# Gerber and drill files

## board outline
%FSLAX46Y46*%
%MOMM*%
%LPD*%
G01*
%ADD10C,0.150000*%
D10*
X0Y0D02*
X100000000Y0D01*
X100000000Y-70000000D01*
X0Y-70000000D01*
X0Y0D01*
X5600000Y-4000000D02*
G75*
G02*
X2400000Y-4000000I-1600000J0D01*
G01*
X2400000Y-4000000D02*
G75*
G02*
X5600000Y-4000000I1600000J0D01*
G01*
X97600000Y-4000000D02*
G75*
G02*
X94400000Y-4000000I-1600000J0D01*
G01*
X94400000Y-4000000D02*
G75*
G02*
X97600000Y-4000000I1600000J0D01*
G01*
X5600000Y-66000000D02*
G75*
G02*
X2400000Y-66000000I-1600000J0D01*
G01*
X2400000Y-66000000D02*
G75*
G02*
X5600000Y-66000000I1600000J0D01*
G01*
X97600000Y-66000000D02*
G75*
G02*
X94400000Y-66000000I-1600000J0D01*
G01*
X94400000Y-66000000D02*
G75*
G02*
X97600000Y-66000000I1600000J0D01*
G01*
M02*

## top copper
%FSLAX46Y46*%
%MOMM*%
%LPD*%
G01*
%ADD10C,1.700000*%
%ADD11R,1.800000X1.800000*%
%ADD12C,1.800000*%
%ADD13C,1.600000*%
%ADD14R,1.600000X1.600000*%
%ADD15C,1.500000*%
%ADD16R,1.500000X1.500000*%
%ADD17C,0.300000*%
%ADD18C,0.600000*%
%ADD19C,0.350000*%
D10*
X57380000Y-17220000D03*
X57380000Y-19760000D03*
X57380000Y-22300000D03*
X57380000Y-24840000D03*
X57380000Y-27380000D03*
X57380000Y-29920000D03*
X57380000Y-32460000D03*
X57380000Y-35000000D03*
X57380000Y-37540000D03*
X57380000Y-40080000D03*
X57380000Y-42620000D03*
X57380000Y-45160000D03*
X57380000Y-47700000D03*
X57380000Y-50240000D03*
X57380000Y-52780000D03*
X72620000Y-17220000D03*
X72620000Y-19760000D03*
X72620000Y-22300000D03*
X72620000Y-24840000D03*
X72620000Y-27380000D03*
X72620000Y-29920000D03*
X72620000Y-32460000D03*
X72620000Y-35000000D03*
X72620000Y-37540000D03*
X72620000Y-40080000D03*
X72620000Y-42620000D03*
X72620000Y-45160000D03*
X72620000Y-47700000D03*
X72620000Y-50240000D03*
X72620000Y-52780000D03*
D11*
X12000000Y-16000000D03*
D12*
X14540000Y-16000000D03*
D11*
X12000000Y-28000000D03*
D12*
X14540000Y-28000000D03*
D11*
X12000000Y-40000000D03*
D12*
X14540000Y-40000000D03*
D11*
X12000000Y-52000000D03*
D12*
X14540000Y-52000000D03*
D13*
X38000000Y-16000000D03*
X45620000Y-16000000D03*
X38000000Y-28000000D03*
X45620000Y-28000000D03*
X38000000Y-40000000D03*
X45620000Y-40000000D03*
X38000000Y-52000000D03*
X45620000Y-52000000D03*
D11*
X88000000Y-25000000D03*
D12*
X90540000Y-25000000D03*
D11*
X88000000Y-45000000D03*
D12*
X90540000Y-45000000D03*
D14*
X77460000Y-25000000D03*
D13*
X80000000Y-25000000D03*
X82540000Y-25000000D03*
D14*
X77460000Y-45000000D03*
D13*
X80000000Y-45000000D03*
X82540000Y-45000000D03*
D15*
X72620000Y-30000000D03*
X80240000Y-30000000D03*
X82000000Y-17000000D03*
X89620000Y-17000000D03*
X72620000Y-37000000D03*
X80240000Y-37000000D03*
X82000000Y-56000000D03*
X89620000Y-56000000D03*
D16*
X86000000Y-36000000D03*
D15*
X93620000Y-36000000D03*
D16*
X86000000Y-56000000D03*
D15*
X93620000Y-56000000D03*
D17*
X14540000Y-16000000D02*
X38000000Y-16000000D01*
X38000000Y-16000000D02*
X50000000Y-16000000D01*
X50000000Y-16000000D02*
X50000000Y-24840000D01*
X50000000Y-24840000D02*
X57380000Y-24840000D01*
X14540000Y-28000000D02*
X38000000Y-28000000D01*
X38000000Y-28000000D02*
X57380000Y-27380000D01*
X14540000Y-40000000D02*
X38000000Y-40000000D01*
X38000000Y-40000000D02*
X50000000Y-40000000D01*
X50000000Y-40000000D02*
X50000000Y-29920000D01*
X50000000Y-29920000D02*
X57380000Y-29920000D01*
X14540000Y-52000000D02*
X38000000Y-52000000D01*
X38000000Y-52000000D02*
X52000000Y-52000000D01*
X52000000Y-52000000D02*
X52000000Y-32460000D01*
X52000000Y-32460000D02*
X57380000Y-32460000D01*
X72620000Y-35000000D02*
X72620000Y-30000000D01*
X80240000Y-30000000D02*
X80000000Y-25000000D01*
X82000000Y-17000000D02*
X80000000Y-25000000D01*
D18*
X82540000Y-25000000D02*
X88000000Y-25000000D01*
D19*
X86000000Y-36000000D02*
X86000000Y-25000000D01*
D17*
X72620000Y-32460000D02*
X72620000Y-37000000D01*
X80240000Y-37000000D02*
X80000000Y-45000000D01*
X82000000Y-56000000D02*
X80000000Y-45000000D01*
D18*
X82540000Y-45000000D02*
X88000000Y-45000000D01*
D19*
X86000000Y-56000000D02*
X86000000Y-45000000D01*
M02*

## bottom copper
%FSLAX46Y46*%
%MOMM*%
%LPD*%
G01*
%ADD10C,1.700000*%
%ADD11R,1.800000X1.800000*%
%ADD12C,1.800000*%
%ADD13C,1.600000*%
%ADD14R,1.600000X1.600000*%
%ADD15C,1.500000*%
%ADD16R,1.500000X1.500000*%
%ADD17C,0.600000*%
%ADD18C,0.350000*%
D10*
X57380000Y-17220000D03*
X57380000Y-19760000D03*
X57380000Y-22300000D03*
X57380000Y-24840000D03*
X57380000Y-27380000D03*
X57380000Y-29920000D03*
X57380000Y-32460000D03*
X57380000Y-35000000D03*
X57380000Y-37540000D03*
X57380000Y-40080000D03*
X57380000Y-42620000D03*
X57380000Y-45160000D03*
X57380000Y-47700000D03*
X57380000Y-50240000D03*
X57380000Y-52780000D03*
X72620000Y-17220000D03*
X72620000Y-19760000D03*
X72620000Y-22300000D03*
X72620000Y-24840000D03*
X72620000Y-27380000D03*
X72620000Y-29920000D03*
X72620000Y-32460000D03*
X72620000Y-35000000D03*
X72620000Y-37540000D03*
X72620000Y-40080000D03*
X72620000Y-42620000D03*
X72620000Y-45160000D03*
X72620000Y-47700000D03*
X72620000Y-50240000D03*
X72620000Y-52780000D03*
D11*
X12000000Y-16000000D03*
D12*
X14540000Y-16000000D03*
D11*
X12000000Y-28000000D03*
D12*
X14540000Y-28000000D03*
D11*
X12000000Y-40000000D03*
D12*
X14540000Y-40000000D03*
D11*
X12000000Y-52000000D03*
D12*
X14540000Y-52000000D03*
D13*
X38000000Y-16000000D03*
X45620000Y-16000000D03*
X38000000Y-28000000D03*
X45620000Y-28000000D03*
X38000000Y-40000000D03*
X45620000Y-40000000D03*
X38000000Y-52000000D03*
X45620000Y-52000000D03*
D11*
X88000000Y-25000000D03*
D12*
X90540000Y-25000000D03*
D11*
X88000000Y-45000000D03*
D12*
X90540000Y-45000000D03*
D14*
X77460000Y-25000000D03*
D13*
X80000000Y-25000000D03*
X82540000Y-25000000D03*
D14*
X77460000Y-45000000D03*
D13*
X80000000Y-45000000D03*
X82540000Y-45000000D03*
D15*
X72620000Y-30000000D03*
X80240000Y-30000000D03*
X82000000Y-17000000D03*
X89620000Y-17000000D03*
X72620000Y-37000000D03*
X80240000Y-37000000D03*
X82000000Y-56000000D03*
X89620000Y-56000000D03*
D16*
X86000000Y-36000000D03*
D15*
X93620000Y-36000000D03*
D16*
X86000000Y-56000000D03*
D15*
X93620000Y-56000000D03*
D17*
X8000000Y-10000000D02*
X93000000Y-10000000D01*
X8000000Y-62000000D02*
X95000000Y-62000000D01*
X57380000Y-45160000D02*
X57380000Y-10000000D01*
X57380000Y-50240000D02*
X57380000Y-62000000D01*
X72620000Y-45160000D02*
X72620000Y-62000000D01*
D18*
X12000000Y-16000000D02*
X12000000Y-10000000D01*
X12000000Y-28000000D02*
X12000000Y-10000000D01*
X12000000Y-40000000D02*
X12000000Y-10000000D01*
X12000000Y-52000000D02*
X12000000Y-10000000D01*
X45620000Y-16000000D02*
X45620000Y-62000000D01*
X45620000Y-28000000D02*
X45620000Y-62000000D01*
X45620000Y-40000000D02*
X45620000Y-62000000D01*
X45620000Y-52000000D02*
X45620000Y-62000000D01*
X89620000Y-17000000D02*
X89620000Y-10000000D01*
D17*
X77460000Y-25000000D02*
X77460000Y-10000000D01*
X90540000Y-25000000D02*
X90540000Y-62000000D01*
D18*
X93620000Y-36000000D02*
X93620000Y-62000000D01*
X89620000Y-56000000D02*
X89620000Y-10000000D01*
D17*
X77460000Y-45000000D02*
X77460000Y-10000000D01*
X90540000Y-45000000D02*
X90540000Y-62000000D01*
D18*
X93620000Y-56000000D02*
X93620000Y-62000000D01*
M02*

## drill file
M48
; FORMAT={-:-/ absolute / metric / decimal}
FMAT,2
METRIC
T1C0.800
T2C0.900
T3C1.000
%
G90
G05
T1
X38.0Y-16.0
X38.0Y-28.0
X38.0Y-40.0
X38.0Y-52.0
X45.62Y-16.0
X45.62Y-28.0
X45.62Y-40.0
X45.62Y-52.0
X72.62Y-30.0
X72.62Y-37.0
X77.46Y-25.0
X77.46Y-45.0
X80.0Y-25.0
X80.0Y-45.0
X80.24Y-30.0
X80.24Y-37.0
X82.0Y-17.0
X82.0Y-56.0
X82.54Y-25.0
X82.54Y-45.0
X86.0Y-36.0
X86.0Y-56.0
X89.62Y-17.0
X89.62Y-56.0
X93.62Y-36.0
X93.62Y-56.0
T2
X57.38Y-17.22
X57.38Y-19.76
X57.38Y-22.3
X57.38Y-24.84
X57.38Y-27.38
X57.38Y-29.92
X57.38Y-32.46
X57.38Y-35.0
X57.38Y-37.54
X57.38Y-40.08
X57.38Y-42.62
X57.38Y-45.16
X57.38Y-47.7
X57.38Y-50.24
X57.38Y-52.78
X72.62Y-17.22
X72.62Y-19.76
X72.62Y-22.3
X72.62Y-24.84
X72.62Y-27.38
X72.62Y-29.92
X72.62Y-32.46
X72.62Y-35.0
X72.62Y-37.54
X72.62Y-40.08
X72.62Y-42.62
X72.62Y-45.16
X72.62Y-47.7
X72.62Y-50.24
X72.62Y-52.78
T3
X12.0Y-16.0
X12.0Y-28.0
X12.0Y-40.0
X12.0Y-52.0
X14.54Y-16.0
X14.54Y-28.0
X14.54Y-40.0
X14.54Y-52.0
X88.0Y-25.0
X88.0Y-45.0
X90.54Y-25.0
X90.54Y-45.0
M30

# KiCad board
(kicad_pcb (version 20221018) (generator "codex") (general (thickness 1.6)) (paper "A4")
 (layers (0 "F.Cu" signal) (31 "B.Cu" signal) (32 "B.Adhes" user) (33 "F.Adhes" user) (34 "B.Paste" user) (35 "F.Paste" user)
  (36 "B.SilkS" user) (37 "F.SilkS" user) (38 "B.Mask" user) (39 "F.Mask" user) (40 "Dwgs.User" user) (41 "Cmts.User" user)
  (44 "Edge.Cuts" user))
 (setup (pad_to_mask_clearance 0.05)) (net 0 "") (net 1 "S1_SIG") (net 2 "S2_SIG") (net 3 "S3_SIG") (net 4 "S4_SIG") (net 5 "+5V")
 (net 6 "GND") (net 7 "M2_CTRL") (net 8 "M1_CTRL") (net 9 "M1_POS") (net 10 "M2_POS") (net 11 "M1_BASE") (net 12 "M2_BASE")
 (gr_rect (start 0 0) (end 100 70) (stroke (width 0.15) (type default)) (fill none) (layer "Edge.Cuts"))
 (gr_circle (center 4 4) (end 5.6 4) (stroke (width 0.15) (type default)) (fill none) (layer "Edge.Cuts"))
 (gr_circle (center 96 4) (end 97.6 4) (stroke (width 0.15) (type default)) (fill none) (layer "Edge.Cuts"))
 (gr_circle (center 4 66) (end 5.6 66) (stroke (width 0.15) (type default)) (fill none) (layer "Edge.Cuts"))
 (gr_circle (center 96 66) (end 97.6 66) (stroke (width 0.15) (type default)) (fill none) (layer "Edge.Cuts"))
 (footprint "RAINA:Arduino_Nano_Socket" (layer "F.Cu") (at 0 0)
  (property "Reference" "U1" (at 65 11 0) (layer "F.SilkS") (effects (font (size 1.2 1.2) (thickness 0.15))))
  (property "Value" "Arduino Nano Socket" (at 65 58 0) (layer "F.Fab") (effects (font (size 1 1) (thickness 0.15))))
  (pad "L1" thru_hole circle (at 57.38 17.22) (size 1.7 1.7) (drill 0.9) (layers "*.Cu" "*.Mask") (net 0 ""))
  (pad "L2" thru_hole circle (at 57.38 19.76) (size 1.7 1.7) (drill 0.9) (layers "*.Cu" "*.Mask") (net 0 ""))
  (pad "L3" thru_hole circle (at 57.38 22.30) (size 1.7 1.7) (drill 0.9) (layers "*.Cu" "*.Mask") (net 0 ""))
  (pad "L4" thru_hole circle (at 57.38 24.84) (size 1.7 1.7) (drill 0.9) (layers "*.Cu" "*.Mask") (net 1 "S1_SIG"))
  (pad "L5" thru_hole circle (at 57.38 27.38) (size 1.7 1.7) (drill 0.9) (layers "*.Cu" "*.Mask") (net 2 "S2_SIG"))
  (pad "L6" thru_hole circle (at 57.38 29.92) (size 1.7 1.7) (drill 0.9) (layers "*.Cu" "*.Mask") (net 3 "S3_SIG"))
  (pad "L7" thru_hole circle (at 57.38 32.46) (size 1.7 1.7) (drill 0.9) (layers "*.Cu" "*.Mask") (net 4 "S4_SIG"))
  (pad "L8" thru_hole circle (at 57.38 35.00) (size 1.7 1.7) (drill 0.9) (layers "*.Cu" "*.Mask") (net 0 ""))
  (pad "L9" thru_hole circle (at 57.38 37.54) (size 1.7 1.7) (drill 0.9) (layers "*.Cu" "*.Mask") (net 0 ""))
  (pad "L10" thru_hole circle (at 57.38 40.08) (size 1.7 1.7) (drill 0.9) (layers "*.Cu" "*.Mask") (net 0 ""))
  (pad "L11" thru_hole circle (at 57.38 42.62) (size 1.7 1.7) (drill 0.9) (layers "*.Cu" "*.Mask") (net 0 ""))
  (pad "L12" thru_hole circle (at 57.38 45.16) (size 1.7 1.7) (drill 0.9) (layers "*.Cu" "*.Mask") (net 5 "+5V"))
  (pad "L13" thru_hole circle (at 57.38 47.70) (size 1.7 1.7) (drill 0.9) (layers "*.Cu" "*.Mask") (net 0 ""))
  (pad "L14" thru_hole circle (at 57.38 50.24) (size 1.7 1.7) (drill 0.9) (layers "*.Cu" "*.Mask") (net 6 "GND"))
  (pad "L15" thru_hole circle (at 57.38 52.78) (size 1.7 1.7) (drill 0.9) (layers "*.Cu" "*.Mask") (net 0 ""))
  (pad "R1" thru_hole circle (at 72.62 17.22) (size 1.7 1.7) (drill 0.9) (layers "*.Cu" "*.Mask") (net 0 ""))
  (pad "R2" thru_hole circle (at 72.62 19.76) (size 1.7 1.7) (drill 0.9) (layers "*.Cu" "*.Mask") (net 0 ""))
  (pad "R3" thru_hole circle (at 72.62 22.30) (size 1.7 1.7) (drill 0.9) (layers "*.Cu" "*.Mask") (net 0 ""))
  (pad "R4" thru_hole circle (at 72.62 24.84) (size 1.7 1.7) (drill 0.9) (layers "*.Cu" "*.Mask") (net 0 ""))
  (pad "R5" thru_hole circle (at 72.62 27.38) (size 1.7 1.7) (drill 0.9) (layers "*.Cu" "*.Mask") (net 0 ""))
  (pad "R6" thru_hole circle (at 72.62 29.92) (size 1.7 1.7) (drill 0.9) (layers "*.Cu" "*.Mask") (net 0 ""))
  (pad "R7" thru_hole circle (at 72.62 32.46) (size 1.7 1.7) (drill 0.9) (layers "*.Cu" "*.Mask") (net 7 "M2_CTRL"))
  (pad "R8" thru_hole circle (at 72.62 35.00) (size 1.7 1.7) (drill 0.9) (layers "*.Cu" "*.Mask") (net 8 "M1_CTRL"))
  (pad "R9" thru_hole circle (at 72.62 37.54) (size 1.7 1.7) (drill 0.9) (layers "*.Cu" "*.Mask") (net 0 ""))
  (pad "R10" thru_hole circle (at 72.62 40.08) (size 1.7 1.7) (drill 0.9) (layers "*.Cu" "*.Mask") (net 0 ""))
  (pad "R11" thru_hole circle (at 72.62 42.62) (size 1.7 1.7) (drill 0.9) (layers "*.Cu" "*.Mask") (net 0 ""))
  (pad "R12" thru_hole circle (at 72.62 45.16) (size 1.7 1.7) (drill 0.9) (layers "*.Cu" "*.Mask") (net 6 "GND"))
  (pad "R13" thru_hole circle (at 72.62 47.70) (size 1.7 1.7) (drill 0.9) (layers "*.Cu" "*.Mask") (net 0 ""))
  (pad "R14" thru_hole circle (at 72.62 50.24) (size 1.7 1.7) (drill 0.9) (layers "*.Cu" "*.Mask") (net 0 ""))
  (pad "R15" thru_hole circle (at 72.62 52.78) (size 1.7 1.7) (drill 0.9) (layers "*.Cu" "*.Mask") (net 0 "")))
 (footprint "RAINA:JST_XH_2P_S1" (layer "F.Cu") (at 0 0)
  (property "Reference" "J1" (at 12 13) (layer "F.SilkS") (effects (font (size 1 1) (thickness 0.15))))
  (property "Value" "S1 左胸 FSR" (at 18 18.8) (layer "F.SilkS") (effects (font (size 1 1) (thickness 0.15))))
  (pad "1" thru_hole rect (at 12 16) (size 1.8 1.8) (drill 1.0) (layers "*.Cu" "*.Mask") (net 5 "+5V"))
  (pad "2" thru_hole circle (at 14.54 16) (size 1.8 1.8) (drill 1.0) (layers "*.Cu" "*.Mask") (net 1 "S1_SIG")))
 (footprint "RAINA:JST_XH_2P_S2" (layer "F.Cu") (at 0 0)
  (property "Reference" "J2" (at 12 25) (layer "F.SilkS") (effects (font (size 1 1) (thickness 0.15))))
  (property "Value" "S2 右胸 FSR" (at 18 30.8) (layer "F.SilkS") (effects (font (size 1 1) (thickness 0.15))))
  (pad "1" thru_hole rect (at 12 28) (size 1.8 1.8) (drill 1.0) (layers "*.Cu" "*.Mask") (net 5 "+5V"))
  (pad "2" thru_hole circle (at 14.54 28) (size 1.8 1.8) (drill 1.0) (layers "*.Cu" "*.Mask") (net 2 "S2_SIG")))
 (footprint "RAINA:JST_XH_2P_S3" (layer "F.Cu") (at 0 0)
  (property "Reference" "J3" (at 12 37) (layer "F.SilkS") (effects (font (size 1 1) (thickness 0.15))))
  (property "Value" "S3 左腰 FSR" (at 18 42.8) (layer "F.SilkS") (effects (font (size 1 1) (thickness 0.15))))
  (pad "1" thru_hole rect (at 12 40) (size 1.8 1.8) (drill 1.0) (layers "*.Cu" "*.Mask") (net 5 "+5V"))
  (pad "2" thru_hole circle (at 14.54 40) (size 1.8 1.8) (drill 1.0) (layers "*.Cu" "*.Mask") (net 3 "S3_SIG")))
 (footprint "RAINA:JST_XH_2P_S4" (layer "F.Cu") (at 0 0)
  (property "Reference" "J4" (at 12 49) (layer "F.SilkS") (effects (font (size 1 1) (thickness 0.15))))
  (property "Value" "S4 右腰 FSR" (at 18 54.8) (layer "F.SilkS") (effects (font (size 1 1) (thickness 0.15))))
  (pad "1" thru_hole rect (at 12 52) (size 1.8 1.8) (drill 1.0) (layers "*.Cu" "*.Mask") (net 5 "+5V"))
  (pad "2" thru_hole circle (at 14.54 52) (size 1.8 1.8) (drill 1.0) (layers "*.Cu" "*.Mask") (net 4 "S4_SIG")))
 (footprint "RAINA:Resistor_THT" (layer "F.Cu") (at 0 0)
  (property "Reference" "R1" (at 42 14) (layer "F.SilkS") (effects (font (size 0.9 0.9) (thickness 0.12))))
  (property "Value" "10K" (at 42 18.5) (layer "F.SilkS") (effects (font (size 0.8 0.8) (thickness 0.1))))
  (pad "1" thru_hole circle (at 38 16) (size 1.6 1.6) (drill 0.8) (layers "*.Cu" "*.Mask") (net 1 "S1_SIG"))
  (pad "2" thru_hole circle (at 45.62 16) (size 1.6 1.6) (drill 0.8) (layers "*.Cu" "*.Mask") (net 6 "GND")))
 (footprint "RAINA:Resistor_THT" (layer "F.Cu") (at 0 0)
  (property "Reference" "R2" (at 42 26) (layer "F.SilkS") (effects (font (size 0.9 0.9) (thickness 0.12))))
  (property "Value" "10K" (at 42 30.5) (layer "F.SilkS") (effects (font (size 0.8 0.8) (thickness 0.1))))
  (pad "1" thru_hole circle (at 38 28) (size 1.6 1.6) (drill 0.8) (layers "*.Cu" "*.Mask") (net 2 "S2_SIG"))
  (pad "2" thru_hole circle (at 45.62 28) (size 1.6 1.6) (drill 0.8) (layers "*.Cu" "*.Mask") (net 6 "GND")))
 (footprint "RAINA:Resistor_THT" (layer "F.Cu") (at 0 0)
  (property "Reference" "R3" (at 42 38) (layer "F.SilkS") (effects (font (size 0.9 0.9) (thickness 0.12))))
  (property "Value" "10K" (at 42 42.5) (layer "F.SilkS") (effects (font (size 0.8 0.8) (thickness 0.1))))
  (pad "1" thru_hole circle (at 38 40) (size 1.6 1.6) (drill 0.8) (layers "*.Cu" "*.Mask") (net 3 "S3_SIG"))
  (pad "2" thru_hole circle (at 45.62 40) (size 1.6 1.6) (drill 0.8) (layers "*.Cu" "*.Mask") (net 6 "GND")))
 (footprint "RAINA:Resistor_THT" (layer "F.Cu") (at 0 0)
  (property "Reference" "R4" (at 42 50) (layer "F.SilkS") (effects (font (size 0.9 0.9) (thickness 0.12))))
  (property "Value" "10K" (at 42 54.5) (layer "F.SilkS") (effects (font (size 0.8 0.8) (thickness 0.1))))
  (pad "1" thru_hole circle (at 38 52) (size 1.6 1.6) (drill 0.8) (layers "*.Cu" "*.Mask") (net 4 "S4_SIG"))
  (pad "2" thru_hole circle (at 45.62 52) (size 1.6 1.6) (drill 0.8) (layers "*.Cu" "*.Mask") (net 6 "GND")))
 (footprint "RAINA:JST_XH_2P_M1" (layer "F.Cu") (at 0 0)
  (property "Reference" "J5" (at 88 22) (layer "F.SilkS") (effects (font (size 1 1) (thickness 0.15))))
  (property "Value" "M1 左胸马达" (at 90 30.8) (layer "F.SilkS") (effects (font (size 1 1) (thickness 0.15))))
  (pad "1" thru_hole rect (at 88 25) (size 1.8 1.8) (drill 1.0) (layers "*.Cu" "*.Mask") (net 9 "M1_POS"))
  (pad "2" thru_hole circle (at 90.54 25) (size 1.8 1.8) (drill 1.0) (layers "*.Cu" "*.Mask") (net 6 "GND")))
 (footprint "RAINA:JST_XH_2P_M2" (layer "F.Cu") (at 0 0)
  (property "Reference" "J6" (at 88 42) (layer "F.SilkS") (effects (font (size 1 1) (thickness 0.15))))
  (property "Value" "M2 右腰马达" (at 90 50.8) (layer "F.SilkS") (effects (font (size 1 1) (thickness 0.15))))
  (pad "1" thru_hole rect (at 88 45) (size 1.8 1.8) (drill 1.0) (layers "*.Cu" "*.Mask") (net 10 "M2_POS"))
  (pad "2" thru_hole circle (at 90.54 45) (size 1.8 1.8) (drill 1.0) (layers "*.Cu" "*.Mask") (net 6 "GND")))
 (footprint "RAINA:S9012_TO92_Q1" (layer "F.Cu") (at 0 0)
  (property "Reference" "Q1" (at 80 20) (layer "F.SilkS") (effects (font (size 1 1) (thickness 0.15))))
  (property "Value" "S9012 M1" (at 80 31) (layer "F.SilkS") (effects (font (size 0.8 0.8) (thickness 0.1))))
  (pad "E" thru_hole rect (at 77.46 25) (size 1.6 1.6) (drill 0.8) (layers "*.Cu" "*.Mask") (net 5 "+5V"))
  (pad "B" thru_hole circle (at 80 25) (size 1.6 1.6) (drill 0.8) (layers "*.Cu" "*.Mask") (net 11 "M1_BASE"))
  (pad "C" thru_hole circle (at 82.54 25) (size 1.6 1.6) (drill 0.8) (layers "*.Cu" "*.Mask") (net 9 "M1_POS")))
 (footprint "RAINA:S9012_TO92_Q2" (layer "F.Cu") (at 0 0)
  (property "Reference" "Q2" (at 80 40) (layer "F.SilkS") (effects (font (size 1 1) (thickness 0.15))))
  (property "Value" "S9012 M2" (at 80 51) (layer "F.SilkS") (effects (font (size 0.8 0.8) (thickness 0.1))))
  (pad "E" thru_hole rect (at 77.46 45) (size 1.6 1.6) (drill 0.8) (layers "*.Cu" "*.Mask") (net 5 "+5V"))
  (pad "B" thru_hole circle (at 80 45) (size 1.6 1.6) (drill 0.8) (layers "*.Cu" "*.Mask") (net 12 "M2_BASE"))
  (pad "C" thru_hole circle (at 82.54 45) (size 1.6 1.6) (drill 0.8) (layers "*.Cu" "*.Mask") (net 10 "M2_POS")))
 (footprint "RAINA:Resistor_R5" (layer "F.Cu") (at 0 0)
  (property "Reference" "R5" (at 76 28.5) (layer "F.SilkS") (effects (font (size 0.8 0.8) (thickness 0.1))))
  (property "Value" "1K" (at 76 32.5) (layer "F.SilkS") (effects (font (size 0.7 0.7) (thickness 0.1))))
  (pad "1" thru_hole circle (at 72.62 30) (size 1.5 1.5) (drill 0.8) (layers "*.Cu" "*.Mask") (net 8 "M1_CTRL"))
  (pad "2" thru_hole circle (at 80.24 30) (size 1.5 1.5) (drill 0.8) (layers "*.Cu" "*.Mask") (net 11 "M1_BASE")))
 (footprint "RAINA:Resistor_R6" (layer "F.Cu") (at 0 0)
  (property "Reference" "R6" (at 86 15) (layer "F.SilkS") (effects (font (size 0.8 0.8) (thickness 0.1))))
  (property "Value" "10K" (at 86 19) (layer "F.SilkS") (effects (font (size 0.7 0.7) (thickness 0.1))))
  (pad "1" thru_hole circle (at 82 17) (size 1.5 1.5) (drill 0.8) (layers "*.Cu" "*.Mask") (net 11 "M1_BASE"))
  (pad "2" thru_hole circle (at 89.62 17) (size 1.5 1.5) (drill 0.8) (layers "*.Cu" "*.Mask") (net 5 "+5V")))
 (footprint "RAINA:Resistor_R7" (layer "F.Cu") (at 0 0)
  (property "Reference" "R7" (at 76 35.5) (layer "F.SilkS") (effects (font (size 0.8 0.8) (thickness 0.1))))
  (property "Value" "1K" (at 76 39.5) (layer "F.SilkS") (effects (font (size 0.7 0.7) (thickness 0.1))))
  (pad "1" thru_hole circle (at 72.62 37) (size 1.5 1.5) (drill 0.8) (layers "*.Cu" "*.Mask") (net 7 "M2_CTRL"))
  (pad "2" thru_hole circle (at 80.24 37) (size 1.5 1.5) (drill 0.8) (layers "*.Cu" "*.Mask") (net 12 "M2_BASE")))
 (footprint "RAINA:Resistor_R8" (layer "F.Cu") (at 0 0)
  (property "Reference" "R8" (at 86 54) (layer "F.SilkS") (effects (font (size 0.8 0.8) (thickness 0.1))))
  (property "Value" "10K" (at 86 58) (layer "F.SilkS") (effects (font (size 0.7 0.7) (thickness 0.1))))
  (pad "1" thru_hole circle (at 82 56) (size 1.5 1.5) (drill 0.8) (layers "*.Cu" "*.Mask") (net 12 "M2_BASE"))
  (pad "2" thru_hole circle (at 89.62 56) (size 1.5 1.5) (drill 0.8) (layers "*.Cu" "*.Mask") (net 5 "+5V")))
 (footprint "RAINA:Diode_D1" (layer "F.Cu") (at 0 0)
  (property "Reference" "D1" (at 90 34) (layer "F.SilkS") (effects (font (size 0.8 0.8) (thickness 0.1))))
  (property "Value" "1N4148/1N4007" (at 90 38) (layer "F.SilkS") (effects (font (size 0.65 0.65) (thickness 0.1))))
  (pad "K" thru_hole rect (at 86 36) (size 1.5 1.5) (drill 0.8) (layers "*.Cu" "*.Mask") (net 9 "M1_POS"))
  (pad "A" thru_hole circle (at 93.62 36) (size 1.5 1.5) (drill 0.8) (layers "*.Cu" "*.Mask") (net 6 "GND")))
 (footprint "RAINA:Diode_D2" (layer "F.Cu") (at 0 0)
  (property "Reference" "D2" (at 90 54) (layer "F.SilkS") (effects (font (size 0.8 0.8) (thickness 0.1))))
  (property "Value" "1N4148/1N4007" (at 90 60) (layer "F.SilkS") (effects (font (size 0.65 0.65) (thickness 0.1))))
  (pad "K" thru_hole rect (at 86 56) (size 1.5 1.5) (drill 0.8) (layers "*.Cu" "*.Mask") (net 10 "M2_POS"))
  (pad "A" thru_hole circle (at 93.62 56) (size 1.5 1.5) (drill 0.8) (layers "*.Cu" "*.Mask") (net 6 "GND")))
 (segment (start 8 10) (end 93 10) (width 0.6) (layer "B.Cu") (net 5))
 (segment (start 8 62) (end 95 62) (width 0.6) (layer "B.Cu") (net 6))
 (segment (start 57.38 45.16) (end 57.38 10) (width 0.6) (layer "B.Cu") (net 5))
 (segment (start 57.38 50.24) (end 57.38 62) (width 0.6) (layer "B.Cu") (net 6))
 (segment (start 72.62 45.16) (end 72.62 62) (width 0.6) (layer "B.Cu") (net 6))
 (segment (start 12 16) (end 12 10) (width 0.35) (layer "B.Cu") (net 5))
 (segment (start 12 28) (end 12 10) (width 0.35) (layer "B.Cu") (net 5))
 (segment (start 12 40) (end 12 10) (width 0.35) (layer "B.Cu") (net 5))
 (segment (start 12 52) (end 12 10) (width 0.35) (layer "B.Cu") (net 5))
 (segment (start 14.54 16) (end 38 16) (width 0.3) (layer "F.Cu") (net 1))
 (segment (start 38 16) (end 50 16) (width 0.3) (layer "F.Cu") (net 1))
 (segment (start 50 16) (end 50 24.84) (width 0.3) (layer "F.Cu") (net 1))
 (segment (start 50 24.84) (end 57.38 24.84) (width 0.3) (layer "F.Cu") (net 1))
 (segment (start 14.54 28) (end 38 28) (width 0.3) (layer "F.Cu") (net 2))
 (segment (start 38 28) (end 57.38 27.38) (width 0.3) (layer "F.Cu") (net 2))
 (segment (start 14.54 40) (end 38 40) (width 0.3) (layer "F.Cu") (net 3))
 (segment (start 38 40) (end 50 40) (width 0.3) (layer "F.Cu") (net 3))
 (segment (start 50 40) (end 50 29.92) (width 0.3) (layer "F.Cu") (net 3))
 (segment (start 50 29.92) (end 57.38 29.92) (width 0.3) (layer "F.Cu") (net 3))
 (segment (start 14.54 52) (end 38 52) (width 0.3) (layer "F.Cu") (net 4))
 (segment (start 38 52) (end 52 52) (width 0.3) (layer "F.Cu") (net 4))
 (segment (start 52 52) (end 52 32.46) (width 0.3) (layer "F.Cu") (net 4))
 (segment (start 52 32.46) (end 57.38 32.46) (width 0.3) (layer "F.Cu") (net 4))
 (segment (start 45.62 16) (end 45.62 62) (width 0.35) (layer "B.Cu") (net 6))
 (segment (start 45.62 28) (end 45.62 62) (width 0.35) (layer "B.Cu") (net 6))
 (segment (start 45.62 40) (end 45.62 62) (width 0.35) (layer "B.Cu") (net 6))
 (segment (start 45.62 52) (end 45.62 62) (width 0.35) (layer "B.Cu") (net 6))
 (segment (start 72.62 35) (end 72.62 30) (width 0.3) (layer "F.Cu") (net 8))
 (segment (start 80.24 30) (end 80 25) (width 0.3) (layer "F.Cu") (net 11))
 (segment (start 82 17) (end 80 25) (width 0.3) (layer "F.Cu") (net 11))
 (segment (start 89.62 17) (end 89.62 10) (width 0.35) (layer "B.Cu") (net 5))
 (segment (start 77.46 25) (end 77.46 10) (width 0.6) (layer "B.Cu") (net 5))
 (segment (start 82.54 25) (end 88 25) (width 0.6) (layer "F.Cu") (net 9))
 (segment (start 86 36) (end 86 25) (width 0.35) (layer "F.Cu") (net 9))
 (segment (start 90.54 25) (end 90.54 62) (width 0.6) (layer "B.Cu") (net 6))
 (segment (start 93.62 36) (end 93.62 62) (width 0.35) (layer "B.Cu") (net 6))
 (segment (start 72.62 32.46) (end 72.62 37) (width 0.3) (layer "F.Cu") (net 7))
 (segment (start 80.24 37) (end 80 45) (width 0.3) (layer "F.Cu") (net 12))
 (segment (start 82 56) (end 80 45) (width 0.3) (layer "F.Cu") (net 12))
 (segment (start 89.62 56) (end 89.62 10) (width 0.35) (layer "B.Cu") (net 5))
 (segment (start 77.46 45) (end 77.46 10) (width 0.6) (layer "B.Cu") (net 5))
 (segment (start 82.54 45) (end 88 45) (width 0.6) (layer "F.Cu") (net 10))
 (segment (start 86 56) (end 86 45) (width 0.35) (layer "F.Cu") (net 10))
 (segment (start 90.54 45) (end 90.54 62) (width 0.6) (layer "B.Cu") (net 6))
 (segment (start 93.62 56) (end 93.62 62) (width 0.35) (layer "B.Cu") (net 6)))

